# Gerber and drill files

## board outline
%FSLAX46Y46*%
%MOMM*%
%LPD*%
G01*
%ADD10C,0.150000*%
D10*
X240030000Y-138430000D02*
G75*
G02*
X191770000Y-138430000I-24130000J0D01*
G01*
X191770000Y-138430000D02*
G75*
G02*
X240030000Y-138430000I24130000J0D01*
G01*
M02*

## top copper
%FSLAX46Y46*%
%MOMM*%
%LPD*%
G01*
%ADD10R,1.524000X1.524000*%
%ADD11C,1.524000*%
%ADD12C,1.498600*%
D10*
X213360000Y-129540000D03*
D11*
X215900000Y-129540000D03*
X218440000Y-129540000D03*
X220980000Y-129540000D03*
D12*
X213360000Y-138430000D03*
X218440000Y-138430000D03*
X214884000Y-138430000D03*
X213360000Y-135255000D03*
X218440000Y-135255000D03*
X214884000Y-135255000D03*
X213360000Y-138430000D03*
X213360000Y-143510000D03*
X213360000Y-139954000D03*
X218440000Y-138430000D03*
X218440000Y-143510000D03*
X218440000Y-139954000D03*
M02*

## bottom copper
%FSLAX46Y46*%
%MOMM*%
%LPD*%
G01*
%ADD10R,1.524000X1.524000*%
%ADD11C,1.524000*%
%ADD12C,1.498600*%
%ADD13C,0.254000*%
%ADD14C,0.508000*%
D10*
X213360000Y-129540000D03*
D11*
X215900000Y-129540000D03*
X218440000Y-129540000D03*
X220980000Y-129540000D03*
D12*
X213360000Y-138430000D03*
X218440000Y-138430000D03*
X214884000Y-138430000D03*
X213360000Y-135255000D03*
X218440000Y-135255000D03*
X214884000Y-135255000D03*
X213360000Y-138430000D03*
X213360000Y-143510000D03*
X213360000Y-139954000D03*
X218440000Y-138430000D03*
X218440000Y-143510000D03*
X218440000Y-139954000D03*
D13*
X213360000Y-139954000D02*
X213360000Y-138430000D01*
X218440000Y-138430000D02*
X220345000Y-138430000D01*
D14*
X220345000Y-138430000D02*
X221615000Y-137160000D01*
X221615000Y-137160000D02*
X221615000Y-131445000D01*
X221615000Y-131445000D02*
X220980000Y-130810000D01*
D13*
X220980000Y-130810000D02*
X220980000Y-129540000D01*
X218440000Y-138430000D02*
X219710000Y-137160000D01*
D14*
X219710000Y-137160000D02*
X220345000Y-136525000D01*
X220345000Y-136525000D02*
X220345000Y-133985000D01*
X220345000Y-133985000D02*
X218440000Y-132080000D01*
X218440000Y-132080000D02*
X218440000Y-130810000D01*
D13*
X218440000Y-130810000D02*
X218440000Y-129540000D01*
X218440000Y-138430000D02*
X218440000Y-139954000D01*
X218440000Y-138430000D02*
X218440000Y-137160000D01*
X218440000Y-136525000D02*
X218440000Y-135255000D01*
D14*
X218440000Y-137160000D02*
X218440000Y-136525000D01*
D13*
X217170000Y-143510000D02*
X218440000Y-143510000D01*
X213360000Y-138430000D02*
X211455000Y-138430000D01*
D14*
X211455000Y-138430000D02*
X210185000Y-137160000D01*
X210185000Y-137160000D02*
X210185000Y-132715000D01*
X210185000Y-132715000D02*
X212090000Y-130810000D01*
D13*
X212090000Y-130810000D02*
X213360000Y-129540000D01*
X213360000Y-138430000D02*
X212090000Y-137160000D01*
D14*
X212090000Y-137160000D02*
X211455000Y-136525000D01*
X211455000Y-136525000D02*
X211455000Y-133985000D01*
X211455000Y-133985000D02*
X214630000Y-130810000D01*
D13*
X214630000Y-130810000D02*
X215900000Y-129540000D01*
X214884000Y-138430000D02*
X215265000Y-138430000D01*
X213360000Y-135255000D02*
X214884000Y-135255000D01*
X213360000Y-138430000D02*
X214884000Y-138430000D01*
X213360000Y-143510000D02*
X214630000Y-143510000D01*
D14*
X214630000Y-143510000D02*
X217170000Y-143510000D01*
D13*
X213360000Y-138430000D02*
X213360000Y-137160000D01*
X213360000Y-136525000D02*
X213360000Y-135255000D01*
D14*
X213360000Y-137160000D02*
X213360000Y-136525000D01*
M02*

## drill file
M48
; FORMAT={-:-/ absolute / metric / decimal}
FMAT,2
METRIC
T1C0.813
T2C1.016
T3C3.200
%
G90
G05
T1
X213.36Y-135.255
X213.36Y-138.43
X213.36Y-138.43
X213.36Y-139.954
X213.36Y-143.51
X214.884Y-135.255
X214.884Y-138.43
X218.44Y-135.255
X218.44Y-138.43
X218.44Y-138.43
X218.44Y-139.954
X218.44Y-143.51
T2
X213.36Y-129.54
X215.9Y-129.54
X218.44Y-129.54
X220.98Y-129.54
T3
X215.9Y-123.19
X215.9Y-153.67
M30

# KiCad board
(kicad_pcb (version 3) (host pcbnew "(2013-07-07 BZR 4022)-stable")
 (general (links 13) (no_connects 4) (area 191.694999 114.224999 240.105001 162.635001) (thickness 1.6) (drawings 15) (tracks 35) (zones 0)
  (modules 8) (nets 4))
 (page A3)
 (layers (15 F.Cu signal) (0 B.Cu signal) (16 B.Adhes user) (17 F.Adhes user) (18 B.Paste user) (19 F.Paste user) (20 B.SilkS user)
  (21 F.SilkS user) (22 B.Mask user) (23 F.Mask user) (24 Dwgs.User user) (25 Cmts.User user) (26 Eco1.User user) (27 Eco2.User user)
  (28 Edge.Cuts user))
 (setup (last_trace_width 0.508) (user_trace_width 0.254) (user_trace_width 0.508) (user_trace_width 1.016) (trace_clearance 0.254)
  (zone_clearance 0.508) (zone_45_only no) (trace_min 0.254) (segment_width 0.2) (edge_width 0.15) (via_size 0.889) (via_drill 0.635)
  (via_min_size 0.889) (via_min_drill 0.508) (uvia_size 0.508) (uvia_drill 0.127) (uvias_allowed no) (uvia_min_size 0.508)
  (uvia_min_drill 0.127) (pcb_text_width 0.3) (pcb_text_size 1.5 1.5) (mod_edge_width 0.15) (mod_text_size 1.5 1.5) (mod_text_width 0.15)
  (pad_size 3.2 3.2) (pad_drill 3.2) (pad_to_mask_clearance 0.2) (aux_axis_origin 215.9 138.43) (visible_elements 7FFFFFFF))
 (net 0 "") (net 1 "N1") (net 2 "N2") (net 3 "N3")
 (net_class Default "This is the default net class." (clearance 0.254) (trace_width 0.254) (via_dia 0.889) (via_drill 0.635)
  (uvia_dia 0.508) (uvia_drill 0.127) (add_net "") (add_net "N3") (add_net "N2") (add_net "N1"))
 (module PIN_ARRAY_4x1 (layer F.Cu) (at 217.17 129.54)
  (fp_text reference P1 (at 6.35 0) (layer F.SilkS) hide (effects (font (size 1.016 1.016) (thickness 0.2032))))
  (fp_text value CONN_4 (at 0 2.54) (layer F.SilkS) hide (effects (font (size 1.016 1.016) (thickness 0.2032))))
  (pad 1 thru_hole rect (at -3.81 0) (size 1.524 1.524) (drill 1.016) (layers *.Cu *.Mask F.SilkS) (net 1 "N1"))
  (pad 2 thru_hole circle (at -1.27 0) (size 1.524 1.524) (drill 1.016) (layers *.Cu *.Mask F.SilkS) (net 1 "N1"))
  (pad 3 thru_hole circle (at 1.27 0) (size 1.524 1.524) (drill 1.016) (layers *.Cu *.Mask F.SilkS) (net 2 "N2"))
  (pad 4 thru_hole circle (at 3.81 0) (size 1.524 1.524) (drill 1.016) (layers *.Cu *.Mask F.SilkS) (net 2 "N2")))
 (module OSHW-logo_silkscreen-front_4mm (layer F.Cu) (at 232.41 138.43 90)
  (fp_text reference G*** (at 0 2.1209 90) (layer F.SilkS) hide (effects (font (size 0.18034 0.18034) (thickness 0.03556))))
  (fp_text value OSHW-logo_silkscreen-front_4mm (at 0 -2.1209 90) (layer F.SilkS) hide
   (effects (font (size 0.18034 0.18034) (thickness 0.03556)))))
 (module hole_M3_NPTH (layer F.Cu) (at 215.9 123.19)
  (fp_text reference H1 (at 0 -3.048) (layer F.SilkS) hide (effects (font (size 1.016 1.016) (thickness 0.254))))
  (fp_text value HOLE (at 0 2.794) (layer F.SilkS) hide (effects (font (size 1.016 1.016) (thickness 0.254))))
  (pad "" np_thru_hole circle (at 0 0) (size 3.2 3.2) (drill 3.2) (layers *.Cu *.Mask F.SilkS)))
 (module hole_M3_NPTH (layer F.Cu) (at 215.9 153.67)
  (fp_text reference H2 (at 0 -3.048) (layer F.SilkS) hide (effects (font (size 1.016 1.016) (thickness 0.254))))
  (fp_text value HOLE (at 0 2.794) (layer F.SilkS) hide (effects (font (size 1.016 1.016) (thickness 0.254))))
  (pad "" np_thru_hole circle (at 0 0) (size 3.2 3.2) (drill 3.2) (layers *.Cu *.Mask F.SilkS)))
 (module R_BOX (layer F.Cu) (at 213.36 138.43)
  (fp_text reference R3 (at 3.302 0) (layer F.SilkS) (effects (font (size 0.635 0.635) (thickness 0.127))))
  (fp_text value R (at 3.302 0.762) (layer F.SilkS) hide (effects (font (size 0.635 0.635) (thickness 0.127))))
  (pad 1 thru_hole circle (at 0 0) (size 1.4986 1.4986) (drill 0.8128) (layers *.Cu *.Mask F.SilkS) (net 1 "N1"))
  (pad 2 thru_hole circle (at 5.08 0) (size 1.4986 1.4986) (drill 0.8128) (layers *.Cu *.Mask F.SilkS) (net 2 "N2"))
  (pad 1 thru_hole circle (at 1.524 0) (size 1.4986 1.4986) (drill 0.8128) (layers *.Cu *.Mask F.SilkS) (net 1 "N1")))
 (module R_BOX (layer F.Cu) (at 213.36 135.255)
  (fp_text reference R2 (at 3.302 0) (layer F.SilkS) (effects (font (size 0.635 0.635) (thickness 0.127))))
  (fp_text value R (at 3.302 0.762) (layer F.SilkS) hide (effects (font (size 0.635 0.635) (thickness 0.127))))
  (pad 1 thru_hole circle (at 0 0) (size 1.4986 1.4986) (drill 0.8128) (layers *.Cu *.Mask F.SilkS) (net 1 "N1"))
  (pad 2 thru_hole circle (at 5.08 0) (size 1.4986 1.4986) (drill 0.8128) (layers *.Cu *.Mask F.SilkS) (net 2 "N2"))
  (pad 1 thru_hole circle (at 1.524 0) (size 1.4986 1.4986) (drill 0.8128) (layers *.Cu *.Mask F.SilkS) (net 1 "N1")))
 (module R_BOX (layer F.Cu) (at 213.36 138.43 270)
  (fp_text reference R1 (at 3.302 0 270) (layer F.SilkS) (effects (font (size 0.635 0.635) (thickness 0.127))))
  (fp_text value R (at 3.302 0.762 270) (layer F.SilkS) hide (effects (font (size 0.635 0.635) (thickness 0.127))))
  (pad 1 thru_hole circle (at 0 0 270) (size 1.4986 1.4986) (drill 0.8128) (layers *.Cu *.Mask F.SilkS) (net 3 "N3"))
  (pad 2 thru_hole circle (at 5.08 0 270) (size 1.4986 1.4986) (drill 0.8128) (layers *.Cu *.Mask F.SilkS) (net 1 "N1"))
  (pad 1 thru_hole circle (at 1.524 0 270) (size 1.4986 1.4986) (drill 0.8128) (layers *.Cu *.Mask F.SilkS) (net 3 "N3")))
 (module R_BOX (layer F.Cu) (at 218.44 138.43 270)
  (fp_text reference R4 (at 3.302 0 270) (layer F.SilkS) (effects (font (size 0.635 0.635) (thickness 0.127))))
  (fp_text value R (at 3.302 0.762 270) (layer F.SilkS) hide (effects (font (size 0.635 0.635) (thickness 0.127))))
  (pad 1 thru_hole circle (at 0 0 270) (size 1.4986 1.4986) (drill 0.8128) (layers *.Cu *.Mask F.SilkS) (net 3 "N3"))
  (pad 2 thru_hole circle (at 5.08 0 270) (size 1.4986 1.4986) (drill 0.8128) (layers *.Cu *.Mask F.SilkS) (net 2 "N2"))
  (pad 1 thru_hole circle (at 1.524 0 270) (size 1.4986 1.4986) (drill 0.8128) (layers *.Cu *.Mask F.SilkS) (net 3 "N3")))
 (gr_circle (center 215.9 138.43) (end 240.03 138.43) (layer Edge.Cuts) (width 0.15))
 (segment (start 213.36 139.954) (end 213.36 138.43) (width 0.254) (layer B.Cu) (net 3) (status C00000))
 (segment (start 218.44 138.43) (end 220.345 138.43) (width 0.254) (layer B.Cu) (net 2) (status 400000))
 (segment (start 220.345 138.43) (end 221.615 137.16) (width 0.508) (layer B.Cu) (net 2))
 (segment (start 221.615 137.16) (end 221.615 131.445) (width 0.508) (layer B.Cu) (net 2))
 (segment (start 221.615 131.445) (end 220.98 130.81) (width 0.508) (layer B.Cu) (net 2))
 (segment (start 220.98 130.81) (end 220.98 129.54) (width 0.254) (layer B.Cu) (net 2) (status 800000))
 (segment (start 218.44 138.43) (end 219.71 137.16) (width 0.254) (layer B.Cu) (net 2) (status 400000))
 (segment (start 219.71 137.16) (end 220.345 136.525) (width 0.508) (layer B.Cu) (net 2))
 (segment (start 220.345 136.525) (end 220.345 133.985) (width 0.508) (layer B.Cu) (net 2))
 (segment (start 220.345 133.985) (end 218.44 132.08) (width 0.508) (layer B.Cu) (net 2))
 (segment (start 218.44 132.08) (end 218.44 130.81) (width 0.508) (layer B.Cu) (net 2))
 (segment (start 218.44 130.81) (end 218.44 129.54) (width 0.254) (layer B.Cu) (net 2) (status 800000))
 (segment (start 218.44 138.43) (end 218.44 139.954) (width 0.254) (layer B.Cu) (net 2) (status C00000))
 (segment (start 218.44 138.43) (end 218.44 137.16) (width 0.254) (layer B.Cu) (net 2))
 (segment (start 218.44 136.525) (end 218.44 135.255) (width 0.254) (layer B.Cu) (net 2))
 (segment (start 218.44 137.16) (end 218.44 136.525) (width 0.508) (layer B.Cu) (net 2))
 (segment (start 217.17 143.51) (end 218.44 143.51) (width 0.254) (layer B.Cu) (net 2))
 (segment (start 213.36 138.43) (end 211.455 138.43) (width 0.254) (layer B.Cu) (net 1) (status 400000))
 (segment (start 211.455 138.43) (end 210.185 137.16) (width 0.508) (layer B.Cu) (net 1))
 (segment (start 210.185 137.16) (end 210.185 132.715) (width 0.508) (layer B.Cu) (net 1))
 (segment (start 210.185 132.715) (end 212.09 130.81) (width 0.508) (layer B.Cu) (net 1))
 (segment (start 212.09 130.81) (end 213.36 129.54) (width 0.254) (layer B.Cu) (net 1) (status 800000))
 (segment (start 213.36 138.43) (end 212.09 137.16) (width 0.254) (layer B.Cu) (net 1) (status 400000))
 (segment (start 212.09 137.16) (end 211.455 136.525) (width 0.508) (layer B.Cu) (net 1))
 (segment (start 211.455 136.525) (end 211.455 133.985) (width 0.508) (layer B.Cu) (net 1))
 (segment (start 211.455 133.985) (end 214.63 130.81) (width 0.508) (layer B.Cu) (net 1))
 (segment (start 214.63 130.81) (end 215.9 129.54) (width 0.254) (layer B.Cu) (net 1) (status 800000))
 (segment (start 214.884 138.43) (end 215.265 138.43) (width 0.254) (layer B.Cu) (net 1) (status C00000))
 (segment (start 213.36 135.255) (end 214.884 135.255) (width 0.254) (layer B.Cu) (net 1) (status C00000))
 (segment (start 213.36 138.43) (end 214.884 138.43) (width 0.254) (layer B.Cu) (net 1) (status C00000))
 (segment (start 213.36 143.51) (end 214.63 143.51) (width 0.254) (layer B.Cu) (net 1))
 (segment (start 214.63 143.51) (end 217.17 143.51) (width 0.508) (layer B.Cu) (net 1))
 (segment (start 213.36 138.43) (end 213.36 137.16) (width 0.254) (layer B.Cu) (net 1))
 (segment (start 213.36 136.525) (end 213.36 135.255) (width 0.254) (layer B.Cu) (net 1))
 (segment (start 213.36 137.16) (end 213.36 136.525) (width 0.508) (layer B.Cu) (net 1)))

